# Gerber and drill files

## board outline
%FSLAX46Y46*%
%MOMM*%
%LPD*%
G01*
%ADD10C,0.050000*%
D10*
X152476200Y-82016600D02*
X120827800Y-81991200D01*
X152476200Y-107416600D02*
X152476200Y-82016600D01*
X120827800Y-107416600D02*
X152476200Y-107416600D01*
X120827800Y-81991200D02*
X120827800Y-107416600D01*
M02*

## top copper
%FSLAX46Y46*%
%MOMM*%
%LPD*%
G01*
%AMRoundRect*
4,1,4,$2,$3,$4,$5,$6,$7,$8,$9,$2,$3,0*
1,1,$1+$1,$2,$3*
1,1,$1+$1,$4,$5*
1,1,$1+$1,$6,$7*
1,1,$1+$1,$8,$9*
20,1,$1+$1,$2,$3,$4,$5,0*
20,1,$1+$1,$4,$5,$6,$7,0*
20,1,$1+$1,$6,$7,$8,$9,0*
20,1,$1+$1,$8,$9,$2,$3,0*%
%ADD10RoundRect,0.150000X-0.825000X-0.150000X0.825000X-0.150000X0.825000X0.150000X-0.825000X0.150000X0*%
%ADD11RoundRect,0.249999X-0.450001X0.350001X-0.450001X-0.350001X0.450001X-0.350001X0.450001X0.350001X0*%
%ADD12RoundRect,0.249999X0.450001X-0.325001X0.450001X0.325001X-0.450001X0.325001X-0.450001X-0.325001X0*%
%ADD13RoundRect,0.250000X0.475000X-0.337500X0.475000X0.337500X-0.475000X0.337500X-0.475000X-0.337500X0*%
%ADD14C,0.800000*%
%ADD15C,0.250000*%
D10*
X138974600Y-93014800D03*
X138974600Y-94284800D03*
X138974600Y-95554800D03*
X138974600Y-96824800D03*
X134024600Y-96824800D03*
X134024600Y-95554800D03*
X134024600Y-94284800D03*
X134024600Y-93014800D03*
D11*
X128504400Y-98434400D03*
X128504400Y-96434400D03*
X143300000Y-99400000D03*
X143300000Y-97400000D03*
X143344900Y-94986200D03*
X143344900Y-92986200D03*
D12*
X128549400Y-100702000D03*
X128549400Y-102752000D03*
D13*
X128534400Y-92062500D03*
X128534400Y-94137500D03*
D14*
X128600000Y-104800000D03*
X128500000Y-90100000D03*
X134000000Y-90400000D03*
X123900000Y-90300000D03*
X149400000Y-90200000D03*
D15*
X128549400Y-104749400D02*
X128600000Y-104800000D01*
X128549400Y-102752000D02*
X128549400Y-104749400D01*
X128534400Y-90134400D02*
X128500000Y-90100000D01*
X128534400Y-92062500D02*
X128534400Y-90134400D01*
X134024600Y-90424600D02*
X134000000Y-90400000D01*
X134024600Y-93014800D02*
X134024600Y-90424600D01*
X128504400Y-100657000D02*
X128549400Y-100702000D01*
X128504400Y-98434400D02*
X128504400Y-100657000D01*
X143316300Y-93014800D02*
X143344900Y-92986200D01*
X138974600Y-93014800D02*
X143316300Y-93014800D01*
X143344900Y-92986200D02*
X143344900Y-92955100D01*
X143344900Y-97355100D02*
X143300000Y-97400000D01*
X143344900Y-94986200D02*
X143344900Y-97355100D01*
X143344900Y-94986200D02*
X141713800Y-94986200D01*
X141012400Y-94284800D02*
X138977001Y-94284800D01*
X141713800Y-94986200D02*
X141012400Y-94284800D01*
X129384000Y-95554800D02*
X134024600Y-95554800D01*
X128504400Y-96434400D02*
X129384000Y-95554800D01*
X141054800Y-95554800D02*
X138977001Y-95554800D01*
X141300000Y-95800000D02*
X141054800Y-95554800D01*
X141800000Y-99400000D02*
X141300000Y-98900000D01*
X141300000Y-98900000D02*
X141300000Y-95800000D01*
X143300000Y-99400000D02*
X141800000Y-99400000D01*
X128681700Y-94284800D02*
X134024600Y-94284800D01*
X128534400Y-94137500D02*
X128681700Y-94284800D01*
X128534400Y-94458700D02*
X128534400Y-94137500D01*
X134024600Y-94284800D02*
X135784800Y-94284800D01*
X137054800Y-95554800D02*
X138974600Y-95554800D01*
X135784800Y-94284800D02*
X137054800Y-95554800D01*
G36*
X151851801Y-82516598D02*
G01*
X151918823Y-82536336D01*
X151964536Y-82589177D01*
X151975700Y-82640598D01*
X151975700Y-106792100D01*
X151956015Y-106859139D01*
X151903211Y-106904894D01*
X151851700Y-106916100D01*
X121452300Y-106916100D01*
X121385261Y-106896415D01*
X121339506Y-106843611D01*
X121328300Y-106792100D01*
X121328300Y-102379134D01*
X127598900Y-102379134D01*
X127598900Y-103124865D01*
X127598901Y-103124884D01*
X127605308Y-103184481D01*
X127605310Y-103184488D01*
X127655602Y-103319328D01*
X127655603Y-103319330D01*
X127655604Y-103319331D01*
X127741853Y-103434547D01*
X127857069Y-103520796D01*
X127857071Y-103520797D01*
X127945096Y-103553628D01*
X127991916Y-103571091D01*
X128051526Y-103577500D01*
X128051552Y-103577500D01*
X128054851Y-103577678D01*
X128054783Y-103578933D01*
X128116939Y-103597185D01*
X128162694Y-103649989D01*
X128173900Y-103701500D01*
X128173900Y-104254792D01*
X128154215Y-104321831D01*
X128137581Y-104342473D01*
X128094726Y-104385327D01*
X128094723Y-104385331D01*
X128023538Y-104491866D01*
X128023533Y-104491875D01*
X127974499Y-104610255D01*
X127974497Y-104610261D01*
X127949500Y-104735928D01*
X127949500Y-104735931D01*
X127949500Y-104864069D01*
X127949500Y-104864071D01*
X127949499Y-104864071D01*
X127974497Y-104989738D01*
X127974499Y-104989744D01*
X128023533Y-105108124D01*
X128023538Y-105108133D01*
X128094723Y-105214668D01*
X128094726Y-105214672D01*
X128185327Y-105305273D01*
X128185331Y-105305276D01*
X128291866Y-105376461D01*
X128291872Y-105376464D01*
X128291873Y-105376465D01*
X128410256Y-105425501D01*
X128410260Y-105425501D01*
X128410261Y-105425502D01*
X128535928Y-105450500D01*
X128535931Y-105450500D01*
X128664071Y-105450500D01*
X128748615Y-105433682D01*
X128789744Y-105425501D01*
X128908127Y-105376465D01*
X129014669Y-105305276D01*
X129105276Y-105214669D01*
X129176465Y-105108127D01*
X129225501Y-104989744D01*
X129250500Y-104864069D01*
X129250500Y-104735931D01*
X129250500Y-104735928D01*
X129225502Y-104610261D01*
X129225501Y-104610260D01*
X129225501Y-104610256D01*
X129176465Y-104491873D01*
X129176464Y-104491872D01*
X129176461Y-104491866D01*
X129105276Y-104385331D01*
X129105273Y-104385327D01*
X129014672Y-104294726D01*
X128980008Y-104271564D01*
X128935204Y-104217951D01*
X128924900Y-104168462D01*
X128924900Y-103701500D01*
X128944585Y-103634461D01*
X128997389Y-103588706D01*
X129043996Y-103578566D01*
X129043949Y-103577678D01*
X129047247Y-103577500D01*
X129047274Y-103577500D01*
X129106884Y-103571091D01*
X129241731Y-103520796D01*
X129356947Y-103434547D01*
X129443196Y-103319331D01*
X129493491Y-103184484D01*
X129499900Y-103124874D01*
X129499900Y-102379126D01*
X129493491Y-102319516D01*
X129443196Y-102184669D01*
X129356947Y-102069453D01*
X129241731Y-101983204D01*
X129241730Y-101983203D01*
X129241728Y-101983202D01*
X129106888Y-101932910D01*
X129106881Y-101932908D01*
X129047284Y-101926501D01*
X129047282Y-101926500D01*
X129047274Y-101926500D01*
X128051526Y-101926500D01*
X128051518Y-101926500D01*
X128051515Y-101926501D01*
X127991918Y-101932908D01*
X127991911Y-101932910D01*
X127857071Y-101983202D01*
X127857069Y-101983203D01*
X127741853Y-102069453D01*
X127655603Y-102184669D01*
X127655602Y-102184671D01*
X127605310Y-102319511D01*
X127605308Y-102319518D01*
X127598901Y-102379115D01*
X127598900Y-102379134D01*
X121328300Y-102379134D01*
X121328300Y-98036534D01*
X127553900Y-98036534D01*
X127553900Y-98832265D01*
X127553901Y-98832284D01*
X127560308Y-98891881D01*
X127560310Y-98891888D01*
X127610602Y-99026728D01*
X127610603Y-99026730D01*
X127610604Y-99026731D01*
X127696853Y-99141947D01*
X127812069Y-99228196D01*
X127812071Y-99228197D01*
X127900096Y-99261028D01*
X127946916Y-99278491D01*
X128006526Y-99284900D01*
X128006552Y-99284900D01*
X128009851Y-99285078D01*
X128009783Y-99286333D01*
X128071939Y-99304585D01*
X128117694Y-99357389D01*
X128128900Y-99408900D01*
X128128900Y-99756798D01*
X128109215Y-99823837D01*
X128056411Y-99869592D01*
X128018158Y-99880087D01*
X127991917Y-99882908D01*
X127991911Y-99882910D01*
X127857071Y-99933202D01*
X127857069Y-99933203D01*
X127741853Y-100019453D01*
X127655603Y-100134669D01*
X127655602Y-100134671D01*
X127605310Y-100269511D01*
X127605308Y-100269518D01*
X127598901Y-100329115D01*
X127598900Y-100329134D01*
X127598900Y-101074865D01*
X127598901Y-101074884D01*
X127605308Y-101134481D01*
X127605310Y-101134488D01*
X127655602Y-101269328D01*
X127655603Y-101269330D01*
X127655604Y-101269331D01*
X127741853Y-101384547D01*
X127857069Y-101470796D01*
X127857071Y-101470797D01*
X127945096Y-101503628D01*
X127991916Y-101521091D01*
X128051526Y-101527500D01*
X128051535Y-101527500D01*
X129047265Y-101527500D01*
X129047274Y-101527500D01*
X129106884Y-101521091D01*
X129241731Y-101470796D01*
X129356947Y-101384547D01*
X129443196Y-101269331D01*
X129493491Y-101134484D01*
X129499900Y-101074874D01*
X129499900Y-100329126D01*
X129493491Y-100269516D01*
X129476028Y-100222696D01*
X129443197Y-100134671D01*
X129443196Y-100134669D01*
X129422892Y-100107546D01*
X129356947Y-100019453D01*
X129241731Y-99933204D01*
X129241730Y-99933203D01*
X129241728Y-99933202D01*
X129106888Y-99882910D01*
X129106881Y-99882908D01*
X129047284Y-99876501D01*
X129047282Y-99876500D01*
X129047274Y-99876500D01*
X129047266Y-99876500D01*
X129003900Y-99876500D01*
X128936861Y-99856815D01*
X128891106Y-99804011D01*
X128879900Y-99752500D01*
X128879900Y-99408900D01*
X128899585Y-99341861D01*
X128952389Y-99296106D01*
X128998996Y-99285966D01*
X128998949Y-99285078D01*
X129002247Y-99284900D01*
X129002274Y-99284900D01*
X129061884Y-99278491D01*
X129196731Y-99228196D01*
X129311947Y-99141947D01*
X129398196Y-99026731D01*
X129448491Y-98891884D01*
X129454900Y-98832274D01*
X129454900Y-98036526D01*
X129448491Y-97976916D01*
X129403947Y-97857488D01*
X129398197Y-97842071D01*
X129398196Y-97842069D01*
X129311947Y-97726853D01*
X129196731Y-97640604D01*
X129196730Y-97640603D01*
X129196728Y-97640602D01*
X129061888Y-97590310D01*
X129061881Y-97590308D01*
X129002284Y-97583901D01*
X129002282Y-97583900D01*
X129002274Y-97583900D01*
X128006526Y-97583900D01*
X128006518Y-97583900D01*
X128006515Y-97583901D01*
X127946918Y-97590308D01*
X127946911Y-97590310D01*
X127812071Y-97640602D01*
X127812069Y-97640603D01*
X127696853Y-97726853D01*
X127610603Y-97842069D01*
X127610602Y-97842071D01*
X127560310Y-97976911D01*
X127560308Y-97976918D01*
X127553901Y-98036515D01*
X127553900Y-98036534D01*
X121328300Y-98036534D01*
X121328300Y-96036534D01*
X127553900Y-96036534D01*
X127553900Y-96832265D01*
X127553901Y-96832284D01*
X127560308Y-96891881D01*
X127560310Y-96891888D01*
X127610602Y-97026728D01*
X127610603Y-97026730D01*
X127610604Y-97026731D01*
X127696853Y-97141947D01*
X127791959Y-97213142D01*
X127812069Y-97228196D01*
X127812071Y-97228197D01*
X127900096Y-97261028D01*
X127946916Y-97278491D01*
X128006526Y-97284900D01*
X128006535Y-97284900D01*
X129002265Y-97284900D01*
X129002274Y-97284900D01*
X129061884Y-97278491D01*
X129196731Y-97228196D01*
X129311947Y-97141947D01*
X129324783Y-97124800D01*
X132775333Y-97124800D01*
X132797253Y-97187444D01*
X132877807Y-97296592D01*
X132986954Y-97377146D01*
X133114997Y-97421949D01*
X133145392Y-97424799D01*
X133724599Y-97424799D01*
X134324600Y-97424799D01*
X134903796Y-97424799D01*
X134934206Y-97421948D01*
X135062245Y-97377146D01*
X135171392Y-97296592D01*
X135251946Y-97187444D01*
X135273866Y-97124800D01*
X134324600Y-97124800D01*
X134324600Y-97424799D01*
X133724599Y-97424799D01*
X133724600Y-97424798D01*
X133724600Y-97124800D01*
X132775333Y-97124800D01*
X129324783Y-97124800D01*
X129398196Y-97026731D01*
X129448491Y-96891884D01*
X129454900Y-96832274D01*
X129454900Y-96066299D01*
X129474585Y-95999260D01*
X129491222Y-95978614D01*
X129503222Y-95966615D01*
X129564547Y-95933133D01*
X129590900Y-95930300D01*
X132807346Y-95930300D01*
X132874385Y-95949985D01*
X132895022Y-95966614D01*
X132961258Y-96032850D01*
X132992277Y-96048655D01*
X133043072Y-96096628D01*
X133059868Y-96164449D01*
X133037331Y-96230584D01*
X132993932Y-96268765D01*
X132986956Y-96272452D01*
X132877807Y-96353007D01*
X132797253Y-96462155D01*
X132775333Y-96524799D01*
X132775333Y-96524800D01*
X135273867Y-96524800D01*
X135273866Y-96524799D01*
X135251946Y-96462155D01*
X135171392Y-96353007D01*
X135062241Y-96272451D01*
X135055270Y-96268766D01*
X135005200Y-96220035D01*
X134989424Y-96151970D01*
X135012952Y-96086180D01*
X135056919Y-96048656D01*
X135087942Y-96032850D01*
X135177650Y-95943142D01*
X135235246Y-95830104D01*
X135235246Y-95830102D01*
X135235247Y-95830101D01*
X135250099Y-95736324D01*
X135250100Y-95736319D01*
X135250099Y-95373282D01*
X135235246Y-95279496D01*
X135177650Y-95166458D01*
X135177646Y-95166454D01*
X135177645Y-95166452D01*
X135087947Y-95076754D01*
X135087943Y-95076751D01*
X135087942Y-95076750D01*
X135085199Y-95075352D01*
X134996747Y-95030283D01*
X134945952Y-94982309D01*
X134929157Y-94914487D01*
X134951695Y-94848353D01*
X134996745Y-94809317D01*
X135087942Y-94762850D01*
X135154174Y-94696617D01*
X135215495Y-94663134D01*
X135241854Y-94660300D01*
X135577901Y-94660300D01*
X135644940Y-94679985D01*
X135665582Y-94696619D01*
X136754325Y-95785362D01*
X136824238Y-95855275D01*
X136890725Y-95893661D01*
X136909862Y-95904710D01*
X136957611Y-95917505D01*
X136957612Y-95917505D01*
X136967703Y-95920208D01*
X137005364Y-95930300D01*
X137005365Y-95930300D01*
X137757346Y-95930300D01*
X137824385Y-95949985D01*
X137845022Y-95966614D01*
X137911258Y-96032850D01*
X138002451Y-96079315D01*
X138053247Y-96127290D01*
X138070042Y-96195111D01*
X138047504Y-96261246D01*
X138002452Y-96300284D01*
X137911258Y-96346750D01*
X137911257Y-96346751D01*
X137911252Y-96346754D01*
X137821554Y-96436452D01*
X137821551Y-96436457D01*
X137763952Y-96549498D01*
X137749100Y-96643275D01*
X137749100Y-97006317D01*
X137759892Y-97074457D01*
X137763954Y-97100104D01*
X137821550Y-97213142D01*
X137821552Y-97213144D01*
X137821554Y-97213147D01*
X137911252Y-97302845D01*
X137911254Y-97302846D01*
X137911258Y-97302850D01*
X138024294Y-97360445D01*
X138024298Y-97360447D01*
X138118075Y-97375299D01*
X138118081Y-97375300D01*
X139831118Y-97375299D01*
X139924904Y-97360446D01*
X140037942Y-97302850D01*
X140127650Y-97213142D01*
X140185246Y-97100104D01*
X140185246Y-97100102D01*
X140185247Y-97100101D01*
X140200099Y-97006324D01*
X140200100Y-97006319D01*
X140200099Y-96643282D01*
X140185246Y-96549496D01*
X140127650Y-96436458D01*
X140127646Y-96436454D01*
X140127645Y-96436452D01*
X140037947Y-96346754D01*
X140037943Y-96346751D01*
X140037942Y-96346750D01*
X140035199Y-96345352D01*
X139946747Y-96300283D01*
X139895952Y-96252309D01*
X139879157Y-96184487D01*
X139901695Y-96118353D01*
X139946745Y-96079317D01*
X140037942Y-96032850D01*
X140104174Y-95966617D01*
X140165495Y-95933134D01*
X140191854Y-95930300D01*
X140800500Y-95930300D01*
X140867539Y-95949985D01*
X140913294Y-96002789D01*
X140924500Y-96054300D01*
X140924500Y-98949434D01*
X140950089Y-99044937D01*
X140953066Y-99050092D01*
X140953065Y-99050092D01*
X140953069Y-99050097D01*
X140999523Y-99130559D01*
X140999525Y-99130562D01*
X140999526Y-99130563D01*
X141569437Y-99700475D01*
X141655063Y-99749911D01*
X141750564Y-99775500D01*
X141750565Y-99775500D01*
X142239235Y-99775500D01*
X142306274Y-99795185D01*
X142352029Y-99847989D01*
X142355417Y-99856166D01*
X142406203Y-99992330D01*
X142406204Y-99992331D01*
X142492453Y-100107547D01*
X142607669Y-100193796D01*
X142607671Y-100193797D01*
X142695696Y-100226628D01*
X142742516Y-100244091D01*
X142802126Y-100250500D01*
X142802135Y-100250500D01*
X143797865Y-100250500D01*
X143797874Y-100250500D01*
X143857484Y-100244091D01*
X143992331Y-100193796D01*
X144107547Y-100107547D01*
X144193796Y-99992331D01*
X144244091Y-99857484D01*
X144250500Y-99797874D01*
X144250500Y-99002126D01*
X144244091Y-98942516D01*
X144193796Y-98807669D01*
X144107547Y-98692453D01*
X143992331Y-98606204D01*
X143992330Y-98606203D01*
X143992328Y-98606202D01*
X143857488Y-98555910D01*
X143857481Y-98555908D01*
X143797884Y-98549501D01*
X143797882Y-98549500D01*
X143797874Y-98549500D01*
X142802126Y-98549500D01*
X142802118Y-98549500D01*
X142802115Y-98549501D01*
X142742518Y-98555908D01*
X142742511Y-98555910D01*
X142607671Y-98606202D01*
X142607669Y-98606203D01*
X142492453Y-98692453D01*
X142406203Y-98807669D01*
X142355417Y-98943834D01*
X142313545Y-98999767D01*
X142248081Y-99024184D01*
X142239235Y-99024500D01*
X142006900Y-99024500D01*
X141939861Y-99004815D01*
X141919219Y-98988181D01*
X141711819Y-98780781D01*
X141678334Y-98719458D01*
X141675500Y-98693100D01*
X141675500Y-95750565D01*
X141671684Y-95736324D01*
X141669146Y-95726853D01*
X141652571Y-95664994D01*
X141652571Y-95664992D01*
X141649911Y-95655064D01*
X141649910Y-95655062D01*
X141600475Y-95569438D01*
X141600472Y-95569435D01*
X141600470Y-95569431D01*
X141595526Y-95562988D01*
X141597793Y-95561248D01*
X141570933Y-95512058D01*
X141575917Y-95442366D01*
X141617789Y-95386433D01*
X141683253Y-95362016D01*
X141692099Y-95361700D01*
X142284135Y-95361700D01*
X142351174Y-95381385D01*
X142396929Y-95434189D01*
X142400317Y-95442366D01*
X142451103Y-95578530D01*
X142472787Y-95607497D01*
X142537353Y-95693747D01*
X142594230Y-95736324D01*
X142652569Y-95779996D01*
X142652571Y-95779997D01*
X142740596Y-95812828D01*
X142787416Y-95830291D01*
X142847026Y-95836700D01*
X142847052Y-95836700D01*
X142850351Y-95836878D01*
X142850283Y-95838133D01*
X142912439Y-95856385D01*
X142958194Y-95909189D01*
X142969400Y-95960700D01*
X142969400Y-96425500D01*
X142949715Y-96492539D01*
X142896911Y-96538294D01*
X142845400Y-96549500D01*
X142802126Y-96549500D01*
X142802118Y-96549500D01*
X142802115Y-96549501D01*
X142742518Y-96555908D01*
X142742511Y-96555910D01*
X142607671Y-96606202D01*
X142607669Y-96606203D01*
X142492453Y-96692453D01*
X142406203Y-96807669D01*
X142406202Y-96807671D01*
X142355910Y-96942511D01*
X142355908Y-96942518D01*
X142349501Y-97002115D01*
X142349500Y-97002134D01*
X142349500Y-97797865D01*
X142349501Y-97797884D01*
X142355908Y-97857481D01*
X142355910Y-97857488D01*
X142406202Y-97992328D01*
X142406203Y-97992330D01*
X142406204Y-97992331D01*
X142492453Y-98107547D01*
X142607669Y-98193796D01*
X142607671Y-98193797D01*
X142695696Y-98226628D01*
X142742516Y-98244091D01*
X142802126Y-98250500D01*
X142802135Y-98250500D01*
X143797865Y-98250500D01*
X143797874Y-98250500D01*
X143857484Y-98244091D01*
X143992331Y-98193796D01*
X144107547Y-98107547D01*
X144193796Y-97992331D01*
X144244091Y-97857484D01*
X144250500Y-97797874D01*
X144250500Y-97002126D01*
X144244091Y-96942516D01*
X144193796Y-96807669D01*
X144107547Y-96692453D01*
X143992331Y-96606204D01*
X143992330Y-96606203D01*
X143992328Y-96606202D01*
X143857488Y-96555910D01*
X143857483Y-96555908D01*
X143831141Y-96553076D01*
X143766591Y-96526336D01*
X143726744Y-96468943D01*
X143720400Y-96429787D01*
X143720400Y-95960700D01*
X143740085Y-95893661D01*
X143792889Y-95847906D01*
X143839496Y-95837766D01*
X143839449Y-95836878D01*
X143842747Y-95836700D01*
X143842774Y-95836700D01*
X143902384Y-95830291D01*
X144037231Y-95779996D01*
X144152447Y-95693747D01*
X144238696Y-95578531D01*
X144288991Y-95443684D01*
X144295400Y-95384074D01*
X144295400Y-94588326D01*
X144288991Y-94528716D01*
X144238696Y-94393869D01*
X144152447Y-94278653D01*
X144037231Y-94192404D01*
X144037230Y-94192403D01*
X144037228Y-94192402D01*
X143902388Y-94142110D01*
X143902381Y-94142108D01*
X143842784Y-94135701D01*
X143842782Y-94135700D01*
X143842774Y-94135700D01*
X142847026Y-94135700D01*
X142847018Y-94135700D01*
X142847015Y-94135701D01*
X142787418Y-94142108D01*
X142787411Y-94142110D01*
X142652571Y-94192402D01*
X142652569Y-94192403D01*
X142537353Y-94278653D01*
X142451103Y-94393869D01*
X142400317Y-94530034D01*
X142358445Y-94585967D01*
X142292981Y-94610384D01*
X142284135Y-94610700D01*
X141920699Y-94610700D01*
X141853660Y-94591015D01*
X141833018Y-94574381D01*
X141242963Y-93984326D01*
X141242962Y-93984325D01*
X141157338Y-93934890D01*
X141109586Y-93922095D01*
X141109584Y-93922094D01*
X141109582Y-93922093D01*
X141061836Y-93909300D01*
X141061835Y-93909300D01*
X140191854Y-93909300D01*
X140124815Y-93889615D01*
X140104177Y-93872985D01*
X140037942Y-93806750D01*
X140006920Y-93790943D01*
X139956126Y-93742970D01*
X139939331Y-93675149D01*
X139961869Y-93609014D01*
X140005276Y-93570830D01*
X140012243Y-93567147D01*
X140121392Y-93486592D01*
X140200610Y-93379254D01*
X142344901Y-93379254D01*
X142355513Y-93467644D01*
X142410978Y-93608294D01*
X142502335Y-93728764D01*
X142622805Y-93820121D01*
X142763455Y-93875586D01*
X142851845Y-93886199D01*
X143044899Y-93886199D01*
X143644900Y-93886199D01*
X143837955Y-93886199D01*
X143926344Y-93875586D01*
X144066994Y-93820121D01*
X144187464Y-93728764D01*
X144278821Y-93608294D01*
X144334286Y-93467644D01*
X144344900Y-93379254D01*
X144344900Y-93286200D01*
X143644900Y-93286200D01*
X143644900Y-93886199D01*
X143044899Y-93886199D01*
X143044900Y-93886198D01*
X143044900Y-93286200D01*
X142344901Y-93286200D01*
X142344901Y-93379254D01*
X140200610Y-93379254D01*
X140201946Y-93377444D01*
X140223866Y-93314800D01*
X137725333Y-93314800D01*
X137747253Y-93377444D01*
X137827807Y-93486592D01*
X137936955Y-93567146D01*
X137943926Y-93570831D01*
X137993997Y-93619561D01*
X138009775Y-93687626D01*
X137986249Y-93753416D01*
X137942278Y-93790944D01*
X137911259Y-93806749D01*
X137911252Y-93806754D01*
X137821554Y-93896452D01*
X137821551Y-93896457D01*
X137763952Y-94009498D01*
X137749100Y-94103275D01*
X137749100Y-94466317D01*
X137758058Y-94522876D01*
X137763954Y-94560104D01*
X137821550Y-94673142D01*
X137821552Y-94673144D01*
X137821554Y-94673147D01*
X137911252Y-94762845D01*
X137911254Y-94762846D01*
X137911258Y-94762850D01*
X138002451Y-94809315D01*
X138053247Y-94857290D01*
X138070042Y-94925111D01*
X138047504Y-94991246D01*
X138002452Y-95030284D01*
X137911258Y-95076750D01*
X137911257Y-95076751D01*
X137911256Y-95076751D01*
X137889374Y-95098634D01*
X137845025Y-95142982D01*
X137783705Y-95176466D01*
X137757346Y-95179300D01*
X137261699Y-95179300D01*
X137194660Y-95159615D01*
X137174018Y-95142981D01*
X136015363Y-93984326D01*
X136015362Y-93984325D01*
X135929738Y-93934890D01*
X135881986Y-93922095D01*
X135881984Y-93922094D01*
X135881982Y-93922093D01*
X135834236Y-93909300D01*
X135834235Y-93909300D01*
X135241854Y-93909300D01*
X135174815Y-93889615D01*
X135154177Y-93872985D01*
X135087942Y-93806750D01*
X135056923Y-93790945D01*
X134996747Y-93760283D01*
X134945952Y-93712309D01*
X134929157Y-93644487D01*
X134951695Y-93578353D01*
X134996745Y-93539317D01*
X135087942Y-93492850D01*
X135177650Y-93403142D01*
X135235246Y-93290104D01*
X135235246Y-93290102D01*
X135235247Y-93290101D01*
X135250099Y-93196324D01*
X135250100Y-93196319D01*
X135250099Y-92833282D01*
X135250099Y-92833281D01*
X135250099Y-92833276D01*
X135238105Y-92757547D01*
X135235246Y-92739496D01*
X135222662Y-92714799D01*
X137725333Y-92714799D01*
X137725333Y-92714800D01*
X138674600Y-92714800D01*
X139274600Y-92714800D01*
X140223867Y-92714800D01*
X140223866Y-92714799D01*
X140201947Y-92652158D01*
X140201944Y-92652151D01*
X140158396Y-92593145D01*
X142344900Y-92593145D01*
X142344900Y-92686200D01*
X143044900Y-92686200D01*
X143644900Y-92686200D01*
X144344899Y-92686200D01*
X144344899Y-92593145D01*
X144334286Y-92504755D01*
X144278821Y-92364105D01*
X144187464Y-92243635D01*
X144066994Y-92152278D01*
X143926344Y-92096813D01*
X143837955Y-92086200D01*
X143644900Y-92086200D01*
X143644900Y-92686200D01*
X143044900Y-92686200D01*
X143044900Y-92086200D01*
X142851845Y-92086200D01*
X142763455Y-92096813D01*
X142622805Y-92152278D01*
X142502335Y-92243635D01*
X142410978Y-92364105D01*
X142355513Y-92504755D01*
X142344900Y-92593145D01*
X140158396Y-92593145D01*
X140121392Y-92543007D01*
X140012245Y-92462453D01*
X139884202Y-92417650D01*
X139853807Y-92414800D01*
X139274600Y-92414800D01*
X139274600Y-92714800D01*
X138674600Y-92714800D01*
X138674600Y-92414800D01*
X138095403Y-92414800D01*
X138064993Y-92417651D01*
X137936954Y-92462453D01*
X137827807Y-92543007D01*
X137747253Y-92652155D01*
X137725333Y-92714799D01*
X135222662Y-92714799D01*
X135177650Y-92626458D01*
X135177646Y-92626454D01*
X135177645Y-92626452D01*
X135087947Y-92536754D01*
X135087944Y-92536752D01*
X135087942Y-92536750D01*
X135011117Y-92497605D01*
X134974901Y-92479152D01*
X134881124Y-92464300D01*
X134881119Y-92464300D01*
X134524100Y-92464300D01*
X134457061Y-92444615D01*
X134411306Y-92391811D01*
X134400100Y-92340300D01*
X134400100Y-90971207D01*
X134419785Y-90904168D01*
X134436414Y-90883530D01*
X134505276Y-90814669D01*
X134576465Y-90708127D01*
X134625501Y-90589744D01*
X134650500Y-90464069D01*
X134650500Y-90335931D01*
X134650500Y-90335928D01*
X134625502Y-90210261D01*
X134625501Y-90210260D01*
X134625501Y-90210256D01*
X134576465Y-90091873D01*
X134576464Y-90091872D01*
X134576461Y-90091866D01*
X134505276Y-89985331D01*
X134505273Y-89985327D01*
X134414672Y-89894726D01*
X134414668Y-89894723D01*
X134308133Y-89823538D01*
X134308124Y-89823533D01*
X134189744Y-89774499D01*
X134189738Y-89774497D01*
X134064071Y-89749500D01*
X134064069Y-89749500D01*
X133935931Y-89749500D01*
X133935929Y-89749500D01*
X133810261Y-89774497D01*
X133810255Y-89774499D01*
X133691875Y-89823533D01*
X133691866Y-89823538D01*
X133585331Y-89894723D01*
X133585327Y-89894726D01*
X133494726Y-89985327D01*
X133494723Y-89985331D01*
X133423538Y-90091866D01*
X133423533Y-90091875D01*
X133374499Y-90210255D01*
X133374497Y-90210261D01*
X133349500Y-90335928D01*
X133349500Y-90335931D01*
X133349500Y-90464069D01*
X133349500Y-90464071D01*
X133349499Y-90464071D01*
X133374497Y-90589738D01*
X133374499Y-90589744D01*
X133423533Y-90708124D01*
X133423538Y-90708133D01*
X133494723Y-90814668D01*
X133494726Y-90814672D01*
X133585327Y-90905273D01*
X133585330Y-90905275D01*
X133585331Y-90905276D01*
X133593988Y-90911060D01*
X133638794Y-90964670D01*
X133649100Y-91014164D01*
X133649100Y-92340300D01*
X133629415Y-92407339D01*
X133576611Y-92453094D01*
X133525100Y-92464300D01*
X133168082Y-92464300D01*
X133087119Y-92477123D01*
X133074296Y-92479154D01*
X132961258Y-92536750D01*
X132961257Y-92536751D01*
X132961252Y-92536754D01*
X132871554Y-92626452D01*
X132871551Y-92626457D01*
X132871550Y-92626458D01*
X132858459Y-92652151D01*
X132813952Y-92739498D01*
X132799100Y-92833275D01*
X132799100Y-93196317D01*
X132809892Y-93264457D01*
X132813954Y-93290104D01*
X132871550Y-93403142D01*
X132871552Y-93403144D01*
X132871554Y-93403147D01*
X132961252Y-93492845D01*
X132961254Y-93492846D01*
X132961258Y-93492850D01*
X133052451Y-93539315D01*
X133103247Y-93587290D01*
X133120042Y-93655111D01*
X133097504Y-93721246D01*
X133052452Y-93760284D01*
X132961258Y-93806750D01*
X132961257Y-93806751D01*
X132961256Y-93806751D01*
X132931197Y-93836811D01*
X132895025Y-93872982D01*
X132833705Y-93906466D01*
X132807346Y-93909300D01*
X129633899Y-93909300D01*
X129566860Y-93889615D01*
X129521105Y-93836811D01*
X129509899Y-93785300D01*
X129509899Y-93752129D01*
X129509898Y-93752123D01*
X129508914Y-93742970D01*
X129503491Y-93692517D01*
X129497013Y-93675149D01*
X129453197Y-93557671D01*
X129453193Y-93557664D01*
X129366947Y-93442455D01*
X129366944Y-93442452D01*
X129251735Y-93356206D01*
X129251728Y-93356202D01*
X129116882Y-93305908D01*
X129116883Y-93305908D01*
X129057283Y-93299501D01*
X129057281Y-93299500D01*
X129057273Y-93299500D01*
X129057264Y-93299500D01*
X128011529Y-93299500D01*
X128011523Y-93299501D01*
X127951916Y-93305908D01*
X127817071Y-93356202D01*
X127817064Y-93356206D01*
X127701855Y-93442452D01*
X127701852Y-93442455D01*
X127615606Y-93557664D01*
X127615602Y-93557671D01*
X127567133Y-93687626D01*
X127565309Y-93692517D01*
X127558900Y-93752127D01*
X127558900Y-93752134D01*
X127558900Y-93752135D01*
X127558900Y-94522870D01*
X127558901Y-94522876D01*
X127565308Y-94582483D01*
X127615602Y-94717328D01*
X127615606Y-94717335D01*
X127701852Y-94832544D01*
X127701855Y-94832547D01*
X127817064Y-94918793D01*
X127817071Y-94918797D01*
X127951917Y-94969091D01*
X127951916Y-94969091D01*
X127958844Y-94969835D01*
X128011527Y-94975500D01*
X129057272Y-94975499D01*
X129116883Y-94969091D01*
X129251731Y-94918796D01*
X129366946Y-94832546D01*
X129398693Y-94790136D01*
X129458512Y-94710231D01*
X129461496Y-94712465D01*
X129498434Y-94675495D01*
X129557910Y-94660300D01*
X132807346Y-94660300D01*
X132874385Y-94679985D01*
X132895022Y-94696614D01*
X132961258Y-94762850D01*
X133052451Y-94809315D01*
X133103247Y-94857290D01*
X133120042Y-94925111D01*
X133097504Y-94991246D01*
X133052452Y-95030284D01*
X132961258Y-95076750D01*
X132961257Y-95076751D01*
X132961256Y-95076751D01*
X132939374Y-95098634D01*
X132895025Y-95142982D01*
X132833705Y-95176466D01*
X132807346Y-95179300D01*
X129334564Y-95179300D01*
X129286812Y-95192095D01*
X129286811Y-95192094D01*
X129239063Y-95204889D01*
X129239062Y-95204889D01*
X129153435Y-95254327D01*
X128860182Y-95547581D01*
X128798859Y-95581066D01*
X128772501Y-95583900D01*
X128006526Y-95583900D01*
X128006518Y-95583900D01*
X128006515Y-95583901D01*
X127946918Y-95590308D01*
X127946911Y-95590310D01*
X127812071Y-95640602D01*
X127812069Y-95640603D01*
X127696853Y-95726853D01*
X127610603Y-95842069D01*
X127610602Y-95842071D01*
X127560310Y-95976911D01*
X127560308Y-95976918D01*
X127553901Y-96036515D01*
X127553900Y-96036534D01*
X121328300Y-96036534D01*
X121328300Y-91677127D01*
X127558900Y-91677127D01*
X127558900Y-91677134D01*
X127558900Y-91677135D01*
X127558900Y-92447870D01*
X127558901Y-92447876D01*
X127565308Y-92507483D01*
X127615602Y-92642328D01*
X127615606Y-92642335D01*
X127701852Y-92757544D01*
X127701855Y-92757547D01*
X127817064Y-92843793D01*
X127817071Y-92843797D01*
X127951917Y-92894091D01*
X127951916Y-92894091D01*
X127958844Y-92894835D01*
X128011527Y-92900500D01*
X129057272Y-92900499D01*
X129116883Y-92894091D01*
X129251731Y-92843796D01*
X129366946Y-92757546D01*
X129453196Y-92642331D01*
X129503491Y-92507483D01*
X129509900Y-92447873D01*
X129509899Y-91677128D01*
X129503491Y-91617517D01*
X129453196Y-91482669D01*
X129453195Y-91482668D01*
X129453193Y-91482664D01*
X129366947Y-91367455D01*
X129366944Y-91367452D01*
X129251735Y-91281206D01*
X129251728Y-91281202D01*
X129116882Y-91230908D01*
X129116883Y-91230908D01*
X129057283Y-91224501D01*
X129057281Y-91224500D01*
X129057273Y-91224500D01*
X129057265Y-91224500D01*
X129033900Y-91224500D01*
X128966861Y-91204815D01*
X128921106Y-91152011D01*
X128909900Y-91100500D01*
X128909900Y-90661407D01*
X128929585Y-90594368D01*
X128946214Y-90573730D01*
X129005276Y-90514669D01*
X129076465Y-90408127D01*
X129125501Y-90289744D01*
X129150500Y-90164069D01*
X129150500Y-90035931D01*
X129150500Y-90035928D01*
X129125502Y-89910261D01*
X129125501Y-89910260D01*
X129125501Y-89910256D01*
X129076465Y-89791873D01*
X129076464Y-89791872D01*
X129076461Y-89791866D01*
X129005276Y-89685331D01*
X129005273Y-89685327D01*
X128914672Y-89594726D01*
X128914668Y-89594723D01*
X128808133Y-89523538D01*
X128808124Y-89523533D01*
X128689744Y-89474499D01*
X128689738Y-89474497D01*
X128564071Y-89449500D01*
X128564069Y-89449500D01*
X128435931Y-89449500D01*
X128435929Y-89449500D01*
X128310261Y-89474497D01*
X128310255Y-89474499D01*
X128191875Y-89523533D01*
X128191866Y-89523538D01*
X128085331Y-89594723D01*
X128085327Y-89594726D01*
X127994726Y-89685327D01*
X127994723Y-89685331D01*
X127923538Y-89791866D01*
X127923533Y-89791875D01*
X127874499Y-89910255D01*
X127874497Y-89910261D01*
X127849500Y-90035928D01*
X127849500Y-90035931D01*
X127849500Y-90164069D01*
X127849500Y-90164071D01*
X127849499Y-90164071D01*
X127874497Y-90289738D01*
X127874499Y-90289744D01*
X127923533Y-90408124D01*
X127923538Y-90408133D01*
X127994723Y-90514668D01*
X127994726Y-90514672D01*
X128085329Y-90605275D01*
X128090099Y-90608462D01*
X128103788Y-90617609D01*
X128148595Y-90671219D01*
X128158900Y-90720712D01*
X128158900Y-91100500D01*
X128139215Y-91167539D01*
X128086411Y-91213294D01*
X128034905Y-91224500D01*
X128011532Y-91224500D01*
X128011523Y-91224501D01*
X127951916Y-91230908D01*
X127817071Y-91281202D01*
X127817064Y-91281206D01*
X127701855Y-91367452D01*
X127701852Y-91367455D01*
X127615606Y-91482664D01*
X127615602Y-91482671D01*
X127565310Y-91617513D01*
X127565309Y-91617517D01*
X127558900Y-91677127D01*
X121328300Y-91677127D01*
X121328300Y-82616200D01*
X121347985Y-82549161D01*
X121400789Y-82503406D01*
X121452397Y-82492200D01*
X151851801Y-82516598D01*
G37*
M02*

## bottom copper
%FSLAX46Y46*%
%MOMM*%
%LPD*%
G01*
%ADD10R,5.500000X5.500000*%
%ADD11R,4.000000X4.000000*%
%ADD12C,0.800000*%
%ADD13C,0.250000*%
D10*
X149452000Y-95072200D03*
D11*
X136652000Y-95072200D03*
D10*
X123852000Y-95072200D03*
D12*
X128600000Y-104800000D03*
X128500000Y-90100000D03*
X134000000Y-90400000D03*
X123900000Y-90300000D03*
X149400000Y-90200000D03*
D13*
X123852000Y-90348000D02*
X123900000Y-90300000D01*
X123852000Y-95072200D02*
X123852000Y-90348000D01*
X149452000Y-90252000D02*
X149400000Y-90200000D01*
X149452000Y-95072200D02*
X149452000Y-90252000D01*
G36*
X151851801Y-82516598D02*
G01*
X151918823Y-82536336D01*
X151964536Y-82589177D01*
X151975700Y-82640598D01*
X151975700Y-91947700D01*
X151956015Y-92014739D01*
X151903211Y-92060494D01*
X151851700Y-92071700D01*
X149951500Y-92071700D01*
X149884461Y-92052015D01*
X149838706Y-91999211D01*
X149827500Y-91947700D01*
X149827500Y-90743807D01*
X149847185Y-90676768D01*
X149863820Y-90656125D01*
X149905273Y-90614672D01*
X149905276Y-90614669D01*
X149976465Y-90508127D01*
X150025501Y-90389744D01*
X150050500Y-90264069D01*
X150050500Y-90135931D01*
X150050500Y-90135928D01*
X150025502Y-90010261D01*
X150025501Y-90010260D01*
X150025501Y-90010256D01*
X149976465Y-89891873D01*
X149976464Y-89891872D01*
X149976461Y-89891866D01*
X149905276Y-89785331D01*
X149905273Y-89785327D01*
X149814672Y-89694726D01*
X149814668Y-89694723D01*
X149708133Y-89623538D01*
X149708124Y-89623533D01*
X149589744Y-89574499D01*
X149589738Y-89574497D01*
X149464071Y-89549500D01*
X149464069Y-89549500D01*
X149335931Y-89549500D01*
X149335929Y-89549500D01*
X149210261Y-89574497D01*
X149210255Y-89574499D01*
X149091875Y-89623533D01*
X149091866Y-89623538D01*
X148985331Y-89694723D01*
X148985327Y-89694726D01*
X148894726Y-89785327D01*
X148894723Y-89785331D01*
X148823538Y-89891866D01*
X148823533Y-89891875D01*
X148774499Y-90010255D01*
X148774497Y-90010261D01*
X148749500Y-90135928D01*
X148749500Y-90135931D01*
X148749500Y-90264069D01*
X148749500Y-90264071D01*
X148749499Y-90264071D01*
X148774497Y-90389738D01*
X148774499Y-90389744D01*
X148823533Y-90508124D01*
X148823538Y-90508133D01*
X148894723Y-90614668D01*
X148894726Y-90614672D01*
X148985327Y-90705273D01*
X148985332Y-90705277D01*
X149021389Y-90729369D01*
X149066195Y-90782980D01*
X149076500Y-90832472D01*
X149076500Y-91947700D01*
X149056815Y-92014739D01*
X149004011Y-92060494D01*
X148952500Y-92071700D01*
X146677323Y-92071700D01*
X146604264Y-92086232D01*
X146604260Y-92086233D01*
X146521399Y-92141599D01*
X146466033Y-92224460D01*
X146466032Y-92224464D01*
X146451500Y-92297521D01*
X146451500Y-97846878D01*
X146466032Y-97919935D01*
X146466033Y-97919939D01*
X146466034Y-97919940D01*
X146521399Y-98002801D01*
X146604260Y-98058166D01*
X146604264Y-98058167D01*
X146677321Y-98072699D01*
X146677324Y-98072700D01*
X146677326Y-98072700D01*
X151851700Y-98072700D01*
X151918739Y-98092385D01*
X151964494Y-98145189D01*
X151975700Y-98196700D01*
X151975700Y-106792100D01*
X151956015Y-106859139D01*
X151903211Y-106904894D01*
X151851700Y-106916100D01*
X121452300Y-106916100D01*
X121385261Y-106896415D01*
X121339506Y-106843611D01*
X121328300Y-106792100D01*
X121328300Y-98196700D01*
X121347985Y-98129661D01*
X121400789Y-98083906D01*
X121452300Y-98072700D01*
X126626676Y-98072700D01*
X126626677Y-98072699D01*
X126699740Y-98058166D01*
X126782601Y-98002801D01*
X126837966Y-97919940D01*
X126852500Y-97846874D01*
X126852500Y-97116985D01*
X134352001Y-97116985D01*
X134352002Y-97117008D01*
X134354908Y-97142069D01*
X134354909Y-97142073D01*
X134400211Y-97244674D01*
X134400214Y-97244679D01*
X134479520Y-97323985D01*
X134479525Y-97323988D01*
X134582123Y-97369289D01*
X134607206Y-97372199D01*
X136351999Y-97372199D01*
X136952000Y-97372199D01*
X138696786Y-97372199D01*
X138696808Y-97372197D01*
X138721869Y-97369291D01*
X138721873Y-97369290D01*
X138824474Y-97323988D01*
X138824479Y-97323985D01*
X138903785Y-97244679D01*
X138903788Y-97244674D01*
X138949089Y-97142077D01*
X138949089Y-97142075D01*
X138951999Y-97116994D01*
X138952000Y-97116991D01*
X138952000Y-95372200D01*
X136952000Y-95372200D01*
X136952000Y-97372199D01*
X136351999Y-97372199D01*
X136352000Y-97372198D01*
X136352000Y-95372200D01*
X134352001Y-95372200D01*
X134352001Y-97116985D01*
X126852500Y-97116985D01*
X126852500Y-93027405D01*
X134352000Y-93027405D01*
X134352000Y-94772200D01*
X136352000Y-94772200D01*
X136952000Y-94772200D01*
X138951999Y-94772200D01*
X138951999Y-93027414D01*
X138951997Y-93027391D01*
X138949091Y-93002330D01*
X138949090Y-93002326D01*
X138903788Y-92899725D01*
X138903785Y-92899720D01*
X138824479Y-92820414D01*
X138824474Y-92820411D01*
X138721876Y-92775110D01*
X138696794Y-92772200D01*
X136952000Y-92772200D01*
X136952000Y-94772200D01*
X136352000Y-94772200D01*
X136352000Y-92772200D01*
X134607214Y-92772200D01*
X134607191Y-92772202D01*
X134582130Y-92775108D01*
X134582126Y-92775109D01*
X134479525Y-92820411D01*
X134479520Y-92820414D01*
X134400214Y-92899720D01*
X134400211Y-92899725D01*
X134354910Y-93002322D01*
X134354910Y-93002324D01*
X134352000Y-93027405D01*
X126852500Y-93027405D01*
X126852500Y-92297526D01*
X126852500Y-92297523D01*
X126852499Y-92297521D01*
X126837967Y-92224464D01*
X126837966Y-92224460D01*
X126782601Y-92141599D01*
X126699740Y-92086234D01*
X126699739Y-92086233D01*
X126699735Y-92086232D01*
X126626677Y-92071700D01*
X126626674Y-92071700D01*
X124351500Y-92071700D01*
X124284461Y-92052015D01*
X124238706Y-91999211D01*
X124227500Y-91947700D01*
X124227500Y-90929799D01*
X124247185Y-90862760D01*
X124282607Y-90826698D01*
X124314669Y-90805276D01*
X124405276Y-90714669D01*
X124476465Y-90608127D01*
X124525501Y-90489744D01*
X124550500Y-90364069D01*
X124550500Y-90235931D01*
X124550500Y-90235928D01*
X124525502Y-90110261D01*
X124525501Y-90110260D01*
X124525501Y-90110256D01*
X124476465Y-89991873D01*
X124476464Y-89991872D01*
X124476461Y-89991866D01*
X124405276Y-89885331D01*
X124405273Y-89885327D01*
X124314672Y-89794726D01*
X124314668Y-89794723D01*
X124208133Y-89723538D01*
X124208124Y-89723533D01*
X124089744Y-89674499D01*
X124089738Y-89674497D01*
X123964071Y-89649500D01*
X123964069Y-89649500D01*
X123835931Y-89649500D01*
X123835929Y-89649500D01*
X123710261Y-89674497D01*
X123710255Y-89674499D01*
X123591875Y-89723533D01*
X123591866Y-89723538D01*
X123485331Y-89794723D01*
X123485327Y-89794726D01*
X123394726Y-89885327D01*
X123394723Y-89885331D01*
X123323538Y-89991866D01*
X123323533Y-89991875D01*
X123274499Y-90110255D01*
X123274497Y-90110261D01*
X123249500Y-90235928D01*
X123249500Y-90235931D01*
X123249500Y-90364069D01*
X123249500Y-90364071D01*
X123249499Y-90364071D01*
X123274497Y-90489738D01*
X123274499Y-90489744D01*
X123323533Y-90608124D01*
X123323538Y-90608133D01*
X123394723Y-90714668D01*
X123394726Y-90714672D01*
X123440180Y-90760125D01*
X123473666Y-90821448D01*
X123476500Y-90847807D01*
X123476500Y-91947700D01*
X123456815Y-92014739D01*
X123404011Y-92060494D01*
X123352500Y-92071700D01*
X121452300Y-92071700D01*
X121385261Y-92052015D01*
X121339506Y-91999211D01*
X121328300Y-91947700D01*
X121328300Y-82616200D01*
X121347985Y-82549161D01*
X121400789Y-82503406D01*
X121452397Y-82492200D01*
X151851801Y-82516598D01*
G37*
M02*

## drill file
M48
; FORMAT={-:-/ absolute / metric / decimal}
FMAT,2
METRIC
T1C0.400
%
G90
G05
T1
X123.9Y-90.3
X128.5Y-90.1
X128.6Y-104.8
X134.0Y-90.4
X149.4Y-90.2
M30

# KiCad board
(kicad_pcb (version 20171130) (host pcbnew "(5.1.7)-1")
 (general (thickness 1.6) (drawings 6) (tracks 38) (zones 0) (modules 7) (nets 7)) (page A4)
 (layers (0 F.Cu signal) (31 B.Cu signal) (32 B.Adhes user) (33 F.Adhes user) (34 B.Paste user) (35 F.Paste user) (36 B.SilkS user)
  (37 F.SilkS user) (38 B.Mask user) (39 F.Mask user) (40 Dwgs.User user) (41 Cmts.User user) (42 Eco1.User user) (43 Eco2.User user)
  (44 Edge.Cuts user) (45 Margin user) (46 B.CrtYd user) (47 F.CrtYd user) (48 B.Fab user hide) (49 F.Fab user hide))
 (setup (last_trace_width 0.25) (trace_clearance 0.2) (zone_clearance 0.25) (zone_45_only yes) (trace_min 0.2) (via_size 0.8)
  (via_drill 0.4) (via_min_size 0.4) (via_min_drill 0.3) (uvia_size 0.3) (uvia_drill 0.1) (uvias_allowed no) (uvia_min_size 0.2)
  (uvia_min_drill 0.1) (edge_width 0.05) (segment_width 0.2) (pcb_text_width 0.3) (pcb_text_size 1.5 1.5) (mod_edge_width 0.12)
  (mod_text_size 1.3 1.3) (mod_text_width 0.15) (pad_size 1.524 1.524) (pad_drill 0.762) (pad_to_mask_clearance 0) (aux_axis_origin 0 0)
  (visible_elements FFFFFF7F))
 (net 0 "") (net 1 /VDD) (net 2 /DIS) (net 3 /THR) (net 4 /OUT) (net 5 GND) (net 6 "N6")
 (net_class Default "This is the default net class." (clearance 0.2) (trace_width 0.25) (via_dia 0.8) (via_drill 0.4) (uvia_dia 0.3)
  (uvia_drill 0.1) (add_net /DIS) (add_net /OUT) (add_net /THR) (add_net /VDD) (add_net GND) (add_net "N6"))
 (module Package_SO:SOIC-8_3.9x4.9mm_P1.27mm (layer F.Cu) (at 136.4996 94.9198)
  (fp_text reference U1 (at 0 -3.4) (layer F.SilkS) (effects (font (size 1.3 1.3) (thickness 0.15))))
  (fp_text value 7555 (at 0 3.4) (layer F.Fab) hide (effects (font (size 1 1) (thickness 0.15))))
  (pad 8 smd roundrect (at 2.475 -1.905) (size 1.95 0.6) (layers F.Cu F.Paste F.Mask) (roundrect_rratio 0.25) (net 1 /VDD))
  (pad 7 smd roundrect (at 2.475 -0.635) (size 1.95 0.6) (layers F.Cu F.Paste F.Mask) (roundrect_rratio 0.25) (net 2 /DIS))
  (pad 6 smd roundrect (at 2.475 0.635) (size 1.95 0.6) (layers F.Cu F.Paste F.Mask) (roundrect_rratio 0.25) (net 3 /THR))
  (pad 5 smd roundrect (at 2.475 1.905) (size 1.95 0.6) (layers F.Cu F.Paste F.Mask) (roundrect_rratio 0.25))
  (pad 4 smd roundrect (at -2.475 1.905) (size 1.95 0.6) (layers F.Cu F.Paste F.Mask) (roundrect_rratio 0.25) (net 1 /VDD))
  (pad 3 smd roundrect (at -2.475 0.635) (size 1.95 0.6) (layers F.Cu F.Paste F.Mask) (roundrect_rratio 0.25) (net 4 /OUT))
  (pad 2 smd roundrect (at -2.475 -0.635) (size 1.95 0.6) (layers F.Cu F.Paste F.Mask) (roundrect_rratio 0.25) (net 3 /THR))
  (pad 1 smd roundrect (at -2.475 -1.905) (size 1.95 0.6) (layers F.Cu F.Paste F.Mask) (roundrect_rratio 0.25) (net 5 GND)))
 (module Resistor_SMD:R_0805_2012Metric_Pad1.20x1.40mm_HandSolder (layer F.Cu) (at 128.5044 97.4344 270)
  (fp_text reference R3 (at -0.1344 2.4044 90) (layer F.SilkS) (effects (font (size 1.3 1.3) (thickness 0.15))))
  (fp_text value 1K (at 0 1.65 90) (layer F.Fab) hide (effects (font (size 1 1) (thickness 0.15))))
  (pad 2 smd roundrect (at 1 0 270) (size 1.2 1.4) (layers F.Cu F.Paste F.Mask) (roundrect_rratio 0.2083325) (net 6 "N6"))
  (pad 1 smd roundrect (at -1 0 270) (size 1.2 1.4) (layers F.Cu F.Paste F.Mask) (roundrect_rratio 0.2083325) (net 4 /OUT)))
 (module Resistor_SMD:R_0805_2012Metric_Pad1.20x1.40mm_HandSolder (layer F.Cu) (at 143.3 98.4 270)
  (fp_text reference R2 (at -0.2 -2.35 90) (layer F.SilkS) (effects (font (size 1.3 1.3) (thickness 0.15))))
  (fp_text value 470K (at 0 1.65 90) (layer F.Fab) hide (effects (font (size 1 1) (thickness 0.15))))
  (pad 2 smd roundrect (at 1 0 270) (size 1.2 1.4) (layers F.Cu F.Paste F.Mask) (roundrect_rratio 0.2083325) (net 3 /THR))
  (pad 1 smd roundrect (at -1 0 270) (size 1.2 1.4) (layers F.Cu F.Paste F.Mask) (roundrect_rratio 0.2083325) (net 2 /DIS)))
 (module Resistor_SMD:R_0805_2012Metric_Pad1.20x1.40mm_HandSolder (layer F.Cu) (at 143.3449 93.9862 270)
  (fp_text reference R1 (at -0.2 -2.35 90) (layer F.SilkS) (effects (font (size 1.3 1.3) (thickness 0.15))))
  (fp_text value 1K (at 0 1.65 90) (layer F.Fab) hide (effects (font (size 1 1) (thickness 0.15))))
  (pad 2 smd roundrect (at 1 0 270) (size 1.2 1.4) (layers F.Cu F.Paste F.Mask) (roundrect_rratio 0.2083325) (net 2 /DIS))
  (pad 1 smd roundrect (at -1 0 270) (size 1.2 1.4) (layers F.Cu F.Paste F.Mask) (roundrect_rratio 0.2083325) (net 1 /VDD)))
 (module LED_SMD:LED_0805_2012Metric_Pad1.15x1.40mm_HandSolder (layer F.Cu) (at 128.5494 101.727 90)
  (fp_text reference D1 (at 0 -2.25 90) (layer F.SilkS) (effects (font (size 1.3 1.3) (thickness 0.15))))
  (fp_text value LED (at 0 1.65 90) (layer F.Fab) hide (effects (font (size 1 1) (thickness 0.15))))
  (pad 2 smd roundrect (at 1.025 0 90) (size 1.15 1.4) (layers F.Cu F.Paste F.Mask) (roundrect_rratio 0.2173904347826087) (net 6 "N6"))
  (pad 1 smd roundrect (at -1.025 0 90) (size 1.15 1.4) (layers F.Cu F.Paste F.Mask) (roundrect_rratio 0.2173904347826087) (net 5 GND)))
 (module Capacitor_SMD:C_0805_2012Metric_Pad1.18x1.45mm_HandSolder (layer F.Cu) (at 128.5344 93.1 90)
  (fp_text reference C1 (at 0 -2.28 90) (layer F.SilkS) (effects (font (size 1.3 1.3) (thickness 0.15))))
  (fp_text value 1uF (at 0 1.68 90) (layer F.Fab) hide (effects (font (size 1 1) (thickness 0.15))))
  (pad 2 smd roundrect (at 1.0375 0 90) (size 1.175 1.45) (layers F.Cu F.Paste F.Mask) (roundrect_rratio 0.2127659574468085) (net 5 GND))
  (pad 1 smd roundrect (at -1.0375 0 90) (size 1.175 1.45) (layers F.Cu F.Paste F.Mask) (roundrect_rratio 0.2127659574468085) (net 3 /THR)))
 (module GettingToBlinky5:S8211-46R (layer B.Cu) (at 136.652 95.0722)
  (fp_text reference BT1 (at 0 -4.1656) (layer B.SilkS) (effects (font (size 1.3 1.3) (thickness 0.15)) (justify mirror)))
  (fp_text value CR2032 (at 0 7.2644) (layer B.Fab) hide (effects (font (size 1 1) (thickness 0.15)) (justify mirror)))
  (pad 1 smd rect (at 12.8 0) (size 5.5 5.5) (layers B.Cu B.Paste B.Mask) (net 1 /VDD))
  (pad 2 smd rect (at 0 0) (size 4 4) (layers B.Cu B.Paste B.Mask) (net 5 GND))
  (pad 1 smd rect (at -12.8 0) (size 5.5 5.5) (layers B.Cu B.Paste B.Mask) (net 1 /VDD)))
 (gr_line (start 152.4762 82.0166) (end 120.8278 81.9912) (layer Edge.Cuts) (width 0.05))
 (gr_line (start 152.4762 107.4166) (end 152.4762 82.0166) (layer Edge.Cuts) (width 0.05))
 (gr_line (start 120.8278 107.4166) (end 152.4762 107.4166) (layer Edge.Cuts) (width 0.05))
 (gr_line (start 120.8278 81.9912) (end 120.8278 107.4166) (layer Edge.Cuts) (width 0.05))
 (via (at 128.6 104.8) (size 0.8) (drill 0.4) (layers F.Cu B.Cu) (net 5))
 (segment (start 128.5494 104.7494) (end 128.6 104.8) (width 0.25) (layer F.Cu) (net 5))
 (segment (start 128.5494 102.752) (end 128.5494 104.7494) (width 0.25) (layer F.Cu) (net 5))
 (via (at 128.5 90.1) (size 0.8) (drill 0.4) (layers F.Cu B.Cu) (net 5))
 (segment (start 128.5344 90.1344) (end 128.5 90.1) (width 0.25) (layer F.Cu) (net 5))
 (segment (start 128.5344 92.0625) (end 128.5344 90.1344) (width 0.25) (layer F.Cu) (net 5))
 (via (at 134 90.4) (size 0.8) (drill 0.4) (layers F.Cu B.Cu) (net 5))
 (segment (start 134.0246 90.4246) (end 134 90.4) (width 0.25) (layer F.Cu) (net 5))
 (segment (start 134.0246 93.0148) (end 134.0246 90.4246) (width 0.25) (layer F.Cu) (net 5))
 (segment (start 128.5044 100.657) (end 128.5494 100.702) (width 0.25) (layer F.Cu) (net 6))
 (segment (start 128.5044 98.4344) (end 128.5044 100.657) (width 0.25) (layer F.Cu) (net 6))
 (segment (start 143.3163 93.0148) (end 143.3449 92.9862) (width 0.25) (layer F.Cu) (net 1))
 (segment (start 138.9746 93.0148) (end 143.3163 93.0148) (width 0.25) (layer F.Cu) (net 1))
 (segment (start 143.3449 92.9862) (end 143.3449 92.9551) (width 0.25) (layer F.Cu) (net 1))
 (via (at 123.9 90.3) (size 0.8) (drill 0.4) (layers F.Cu B.Cu) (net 1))
 (segment (start 123.852 90.348) (end 123.9 90.3) (width 0.25) (layer B.Cu) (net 1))
 (segment (start 123.852 95.0722) (end 123.852 90.348) (width 0.25) (layer B.Cu) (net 1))
 (via (at 149.4 90.2) (size 0.8) (drill 0.4) (layers F.Cu B.Cu) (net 1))
 (segment (start 149.452 90.252) (end 149.4 90.2) (width 0.25) (layer B.Cu) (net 1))
 (segment (start 149.452 95.0722) (end 149.452 90.252) (width 0.25) (layer B.Cu) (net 1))
 (segment (start 143.3449 97.3551) (end 143.3 97.4) (width 0.25) (layer F.Cu) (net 2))
 (segment (start 143.3449 94.9862) (end 143.3449 97.3551) (width 0.25) (layer F.Cu) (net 2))
 (segment (start 143.3449 94.9862) (end 141.7138 94.9862) (width 0.25) (layer F.Cu) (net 2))
 (segment (start 141.0124 94.2848) (end 138.977001 94.2848) (width 0.25) (layer F.Cu) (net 2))
 (segment (start 141.7138 94.9862) (end 141.0124 94.2848) (width 0.25) (layer F.Cu) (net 2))
 (segment (start 129.384 95.5548) (end 134.0246 95.5548) (width 0.25) (layer F.Cu) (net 4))
 (segment (start 128.5044 96.4344) (end 129.384 95.5548) (width 0.25) (layer F.Cu) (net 4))
 (segment (start 141.0548 95.5548) (end 138.977001 95.5548) (width 0.25) (layer F.Cu) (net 3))
 (segment (start 141.3 95.8) (end 141.0548 95.5548) (width 0.25) (layer F.Cu) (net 3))
 (segment (start 141.8 99.4) (end 141.3 98.9) (width 0.25) (layer F.Cu) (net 3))
 (segment (start 141.3 98.9) (end 141.3 95.8) (width 0.25) (layer F.Cu) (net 3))
 (segment (start 143.3 99.4) (end 141.8 99.4) (width 0.25) (layer F.Cu) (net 3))
 (segment (start 128.6817 94.2848) (end 134.0246 94.2848) (width 0.25) (layer F.Cu) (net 3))
 (segment (start 128.5344 94.1375) (end 128.6817 94.2848) (width 0.25) (layer F.Cu) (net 3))
 (segment (start 128.5344 94.4587) (end 128.5344 94.1375) (width 0.25) (layer F.Cu) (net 3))
 (segment (start 134.0246 94.2848) (end 135.7848 94.2848) (width 0.25) (layer F.Cu) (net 3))
 (segment (start 137.0548 95.5548) (end 138.9746 95.5548) (width 0.25) (layer F.Cu) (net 3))
 (segment (start 135.7848 94.2848) (end 137.0548 95.5548) (width 0.25) (layer F.Cu) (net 3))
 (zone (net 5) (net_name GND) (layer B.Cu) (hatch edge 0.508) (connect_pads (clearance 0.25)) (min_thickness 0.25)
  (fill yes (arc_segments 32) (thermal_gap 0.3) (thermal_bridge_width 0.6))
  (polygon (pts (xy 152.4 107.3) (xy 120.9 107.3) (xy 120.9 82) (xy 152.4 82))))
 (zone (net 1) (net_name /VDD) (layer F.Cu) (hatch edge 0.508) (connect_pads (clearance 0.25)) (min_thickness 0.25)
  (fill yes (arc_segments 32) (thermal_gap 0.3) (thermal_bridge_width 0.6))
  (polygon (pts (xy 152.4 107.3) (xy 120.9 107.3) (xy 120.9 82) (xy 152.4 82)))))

